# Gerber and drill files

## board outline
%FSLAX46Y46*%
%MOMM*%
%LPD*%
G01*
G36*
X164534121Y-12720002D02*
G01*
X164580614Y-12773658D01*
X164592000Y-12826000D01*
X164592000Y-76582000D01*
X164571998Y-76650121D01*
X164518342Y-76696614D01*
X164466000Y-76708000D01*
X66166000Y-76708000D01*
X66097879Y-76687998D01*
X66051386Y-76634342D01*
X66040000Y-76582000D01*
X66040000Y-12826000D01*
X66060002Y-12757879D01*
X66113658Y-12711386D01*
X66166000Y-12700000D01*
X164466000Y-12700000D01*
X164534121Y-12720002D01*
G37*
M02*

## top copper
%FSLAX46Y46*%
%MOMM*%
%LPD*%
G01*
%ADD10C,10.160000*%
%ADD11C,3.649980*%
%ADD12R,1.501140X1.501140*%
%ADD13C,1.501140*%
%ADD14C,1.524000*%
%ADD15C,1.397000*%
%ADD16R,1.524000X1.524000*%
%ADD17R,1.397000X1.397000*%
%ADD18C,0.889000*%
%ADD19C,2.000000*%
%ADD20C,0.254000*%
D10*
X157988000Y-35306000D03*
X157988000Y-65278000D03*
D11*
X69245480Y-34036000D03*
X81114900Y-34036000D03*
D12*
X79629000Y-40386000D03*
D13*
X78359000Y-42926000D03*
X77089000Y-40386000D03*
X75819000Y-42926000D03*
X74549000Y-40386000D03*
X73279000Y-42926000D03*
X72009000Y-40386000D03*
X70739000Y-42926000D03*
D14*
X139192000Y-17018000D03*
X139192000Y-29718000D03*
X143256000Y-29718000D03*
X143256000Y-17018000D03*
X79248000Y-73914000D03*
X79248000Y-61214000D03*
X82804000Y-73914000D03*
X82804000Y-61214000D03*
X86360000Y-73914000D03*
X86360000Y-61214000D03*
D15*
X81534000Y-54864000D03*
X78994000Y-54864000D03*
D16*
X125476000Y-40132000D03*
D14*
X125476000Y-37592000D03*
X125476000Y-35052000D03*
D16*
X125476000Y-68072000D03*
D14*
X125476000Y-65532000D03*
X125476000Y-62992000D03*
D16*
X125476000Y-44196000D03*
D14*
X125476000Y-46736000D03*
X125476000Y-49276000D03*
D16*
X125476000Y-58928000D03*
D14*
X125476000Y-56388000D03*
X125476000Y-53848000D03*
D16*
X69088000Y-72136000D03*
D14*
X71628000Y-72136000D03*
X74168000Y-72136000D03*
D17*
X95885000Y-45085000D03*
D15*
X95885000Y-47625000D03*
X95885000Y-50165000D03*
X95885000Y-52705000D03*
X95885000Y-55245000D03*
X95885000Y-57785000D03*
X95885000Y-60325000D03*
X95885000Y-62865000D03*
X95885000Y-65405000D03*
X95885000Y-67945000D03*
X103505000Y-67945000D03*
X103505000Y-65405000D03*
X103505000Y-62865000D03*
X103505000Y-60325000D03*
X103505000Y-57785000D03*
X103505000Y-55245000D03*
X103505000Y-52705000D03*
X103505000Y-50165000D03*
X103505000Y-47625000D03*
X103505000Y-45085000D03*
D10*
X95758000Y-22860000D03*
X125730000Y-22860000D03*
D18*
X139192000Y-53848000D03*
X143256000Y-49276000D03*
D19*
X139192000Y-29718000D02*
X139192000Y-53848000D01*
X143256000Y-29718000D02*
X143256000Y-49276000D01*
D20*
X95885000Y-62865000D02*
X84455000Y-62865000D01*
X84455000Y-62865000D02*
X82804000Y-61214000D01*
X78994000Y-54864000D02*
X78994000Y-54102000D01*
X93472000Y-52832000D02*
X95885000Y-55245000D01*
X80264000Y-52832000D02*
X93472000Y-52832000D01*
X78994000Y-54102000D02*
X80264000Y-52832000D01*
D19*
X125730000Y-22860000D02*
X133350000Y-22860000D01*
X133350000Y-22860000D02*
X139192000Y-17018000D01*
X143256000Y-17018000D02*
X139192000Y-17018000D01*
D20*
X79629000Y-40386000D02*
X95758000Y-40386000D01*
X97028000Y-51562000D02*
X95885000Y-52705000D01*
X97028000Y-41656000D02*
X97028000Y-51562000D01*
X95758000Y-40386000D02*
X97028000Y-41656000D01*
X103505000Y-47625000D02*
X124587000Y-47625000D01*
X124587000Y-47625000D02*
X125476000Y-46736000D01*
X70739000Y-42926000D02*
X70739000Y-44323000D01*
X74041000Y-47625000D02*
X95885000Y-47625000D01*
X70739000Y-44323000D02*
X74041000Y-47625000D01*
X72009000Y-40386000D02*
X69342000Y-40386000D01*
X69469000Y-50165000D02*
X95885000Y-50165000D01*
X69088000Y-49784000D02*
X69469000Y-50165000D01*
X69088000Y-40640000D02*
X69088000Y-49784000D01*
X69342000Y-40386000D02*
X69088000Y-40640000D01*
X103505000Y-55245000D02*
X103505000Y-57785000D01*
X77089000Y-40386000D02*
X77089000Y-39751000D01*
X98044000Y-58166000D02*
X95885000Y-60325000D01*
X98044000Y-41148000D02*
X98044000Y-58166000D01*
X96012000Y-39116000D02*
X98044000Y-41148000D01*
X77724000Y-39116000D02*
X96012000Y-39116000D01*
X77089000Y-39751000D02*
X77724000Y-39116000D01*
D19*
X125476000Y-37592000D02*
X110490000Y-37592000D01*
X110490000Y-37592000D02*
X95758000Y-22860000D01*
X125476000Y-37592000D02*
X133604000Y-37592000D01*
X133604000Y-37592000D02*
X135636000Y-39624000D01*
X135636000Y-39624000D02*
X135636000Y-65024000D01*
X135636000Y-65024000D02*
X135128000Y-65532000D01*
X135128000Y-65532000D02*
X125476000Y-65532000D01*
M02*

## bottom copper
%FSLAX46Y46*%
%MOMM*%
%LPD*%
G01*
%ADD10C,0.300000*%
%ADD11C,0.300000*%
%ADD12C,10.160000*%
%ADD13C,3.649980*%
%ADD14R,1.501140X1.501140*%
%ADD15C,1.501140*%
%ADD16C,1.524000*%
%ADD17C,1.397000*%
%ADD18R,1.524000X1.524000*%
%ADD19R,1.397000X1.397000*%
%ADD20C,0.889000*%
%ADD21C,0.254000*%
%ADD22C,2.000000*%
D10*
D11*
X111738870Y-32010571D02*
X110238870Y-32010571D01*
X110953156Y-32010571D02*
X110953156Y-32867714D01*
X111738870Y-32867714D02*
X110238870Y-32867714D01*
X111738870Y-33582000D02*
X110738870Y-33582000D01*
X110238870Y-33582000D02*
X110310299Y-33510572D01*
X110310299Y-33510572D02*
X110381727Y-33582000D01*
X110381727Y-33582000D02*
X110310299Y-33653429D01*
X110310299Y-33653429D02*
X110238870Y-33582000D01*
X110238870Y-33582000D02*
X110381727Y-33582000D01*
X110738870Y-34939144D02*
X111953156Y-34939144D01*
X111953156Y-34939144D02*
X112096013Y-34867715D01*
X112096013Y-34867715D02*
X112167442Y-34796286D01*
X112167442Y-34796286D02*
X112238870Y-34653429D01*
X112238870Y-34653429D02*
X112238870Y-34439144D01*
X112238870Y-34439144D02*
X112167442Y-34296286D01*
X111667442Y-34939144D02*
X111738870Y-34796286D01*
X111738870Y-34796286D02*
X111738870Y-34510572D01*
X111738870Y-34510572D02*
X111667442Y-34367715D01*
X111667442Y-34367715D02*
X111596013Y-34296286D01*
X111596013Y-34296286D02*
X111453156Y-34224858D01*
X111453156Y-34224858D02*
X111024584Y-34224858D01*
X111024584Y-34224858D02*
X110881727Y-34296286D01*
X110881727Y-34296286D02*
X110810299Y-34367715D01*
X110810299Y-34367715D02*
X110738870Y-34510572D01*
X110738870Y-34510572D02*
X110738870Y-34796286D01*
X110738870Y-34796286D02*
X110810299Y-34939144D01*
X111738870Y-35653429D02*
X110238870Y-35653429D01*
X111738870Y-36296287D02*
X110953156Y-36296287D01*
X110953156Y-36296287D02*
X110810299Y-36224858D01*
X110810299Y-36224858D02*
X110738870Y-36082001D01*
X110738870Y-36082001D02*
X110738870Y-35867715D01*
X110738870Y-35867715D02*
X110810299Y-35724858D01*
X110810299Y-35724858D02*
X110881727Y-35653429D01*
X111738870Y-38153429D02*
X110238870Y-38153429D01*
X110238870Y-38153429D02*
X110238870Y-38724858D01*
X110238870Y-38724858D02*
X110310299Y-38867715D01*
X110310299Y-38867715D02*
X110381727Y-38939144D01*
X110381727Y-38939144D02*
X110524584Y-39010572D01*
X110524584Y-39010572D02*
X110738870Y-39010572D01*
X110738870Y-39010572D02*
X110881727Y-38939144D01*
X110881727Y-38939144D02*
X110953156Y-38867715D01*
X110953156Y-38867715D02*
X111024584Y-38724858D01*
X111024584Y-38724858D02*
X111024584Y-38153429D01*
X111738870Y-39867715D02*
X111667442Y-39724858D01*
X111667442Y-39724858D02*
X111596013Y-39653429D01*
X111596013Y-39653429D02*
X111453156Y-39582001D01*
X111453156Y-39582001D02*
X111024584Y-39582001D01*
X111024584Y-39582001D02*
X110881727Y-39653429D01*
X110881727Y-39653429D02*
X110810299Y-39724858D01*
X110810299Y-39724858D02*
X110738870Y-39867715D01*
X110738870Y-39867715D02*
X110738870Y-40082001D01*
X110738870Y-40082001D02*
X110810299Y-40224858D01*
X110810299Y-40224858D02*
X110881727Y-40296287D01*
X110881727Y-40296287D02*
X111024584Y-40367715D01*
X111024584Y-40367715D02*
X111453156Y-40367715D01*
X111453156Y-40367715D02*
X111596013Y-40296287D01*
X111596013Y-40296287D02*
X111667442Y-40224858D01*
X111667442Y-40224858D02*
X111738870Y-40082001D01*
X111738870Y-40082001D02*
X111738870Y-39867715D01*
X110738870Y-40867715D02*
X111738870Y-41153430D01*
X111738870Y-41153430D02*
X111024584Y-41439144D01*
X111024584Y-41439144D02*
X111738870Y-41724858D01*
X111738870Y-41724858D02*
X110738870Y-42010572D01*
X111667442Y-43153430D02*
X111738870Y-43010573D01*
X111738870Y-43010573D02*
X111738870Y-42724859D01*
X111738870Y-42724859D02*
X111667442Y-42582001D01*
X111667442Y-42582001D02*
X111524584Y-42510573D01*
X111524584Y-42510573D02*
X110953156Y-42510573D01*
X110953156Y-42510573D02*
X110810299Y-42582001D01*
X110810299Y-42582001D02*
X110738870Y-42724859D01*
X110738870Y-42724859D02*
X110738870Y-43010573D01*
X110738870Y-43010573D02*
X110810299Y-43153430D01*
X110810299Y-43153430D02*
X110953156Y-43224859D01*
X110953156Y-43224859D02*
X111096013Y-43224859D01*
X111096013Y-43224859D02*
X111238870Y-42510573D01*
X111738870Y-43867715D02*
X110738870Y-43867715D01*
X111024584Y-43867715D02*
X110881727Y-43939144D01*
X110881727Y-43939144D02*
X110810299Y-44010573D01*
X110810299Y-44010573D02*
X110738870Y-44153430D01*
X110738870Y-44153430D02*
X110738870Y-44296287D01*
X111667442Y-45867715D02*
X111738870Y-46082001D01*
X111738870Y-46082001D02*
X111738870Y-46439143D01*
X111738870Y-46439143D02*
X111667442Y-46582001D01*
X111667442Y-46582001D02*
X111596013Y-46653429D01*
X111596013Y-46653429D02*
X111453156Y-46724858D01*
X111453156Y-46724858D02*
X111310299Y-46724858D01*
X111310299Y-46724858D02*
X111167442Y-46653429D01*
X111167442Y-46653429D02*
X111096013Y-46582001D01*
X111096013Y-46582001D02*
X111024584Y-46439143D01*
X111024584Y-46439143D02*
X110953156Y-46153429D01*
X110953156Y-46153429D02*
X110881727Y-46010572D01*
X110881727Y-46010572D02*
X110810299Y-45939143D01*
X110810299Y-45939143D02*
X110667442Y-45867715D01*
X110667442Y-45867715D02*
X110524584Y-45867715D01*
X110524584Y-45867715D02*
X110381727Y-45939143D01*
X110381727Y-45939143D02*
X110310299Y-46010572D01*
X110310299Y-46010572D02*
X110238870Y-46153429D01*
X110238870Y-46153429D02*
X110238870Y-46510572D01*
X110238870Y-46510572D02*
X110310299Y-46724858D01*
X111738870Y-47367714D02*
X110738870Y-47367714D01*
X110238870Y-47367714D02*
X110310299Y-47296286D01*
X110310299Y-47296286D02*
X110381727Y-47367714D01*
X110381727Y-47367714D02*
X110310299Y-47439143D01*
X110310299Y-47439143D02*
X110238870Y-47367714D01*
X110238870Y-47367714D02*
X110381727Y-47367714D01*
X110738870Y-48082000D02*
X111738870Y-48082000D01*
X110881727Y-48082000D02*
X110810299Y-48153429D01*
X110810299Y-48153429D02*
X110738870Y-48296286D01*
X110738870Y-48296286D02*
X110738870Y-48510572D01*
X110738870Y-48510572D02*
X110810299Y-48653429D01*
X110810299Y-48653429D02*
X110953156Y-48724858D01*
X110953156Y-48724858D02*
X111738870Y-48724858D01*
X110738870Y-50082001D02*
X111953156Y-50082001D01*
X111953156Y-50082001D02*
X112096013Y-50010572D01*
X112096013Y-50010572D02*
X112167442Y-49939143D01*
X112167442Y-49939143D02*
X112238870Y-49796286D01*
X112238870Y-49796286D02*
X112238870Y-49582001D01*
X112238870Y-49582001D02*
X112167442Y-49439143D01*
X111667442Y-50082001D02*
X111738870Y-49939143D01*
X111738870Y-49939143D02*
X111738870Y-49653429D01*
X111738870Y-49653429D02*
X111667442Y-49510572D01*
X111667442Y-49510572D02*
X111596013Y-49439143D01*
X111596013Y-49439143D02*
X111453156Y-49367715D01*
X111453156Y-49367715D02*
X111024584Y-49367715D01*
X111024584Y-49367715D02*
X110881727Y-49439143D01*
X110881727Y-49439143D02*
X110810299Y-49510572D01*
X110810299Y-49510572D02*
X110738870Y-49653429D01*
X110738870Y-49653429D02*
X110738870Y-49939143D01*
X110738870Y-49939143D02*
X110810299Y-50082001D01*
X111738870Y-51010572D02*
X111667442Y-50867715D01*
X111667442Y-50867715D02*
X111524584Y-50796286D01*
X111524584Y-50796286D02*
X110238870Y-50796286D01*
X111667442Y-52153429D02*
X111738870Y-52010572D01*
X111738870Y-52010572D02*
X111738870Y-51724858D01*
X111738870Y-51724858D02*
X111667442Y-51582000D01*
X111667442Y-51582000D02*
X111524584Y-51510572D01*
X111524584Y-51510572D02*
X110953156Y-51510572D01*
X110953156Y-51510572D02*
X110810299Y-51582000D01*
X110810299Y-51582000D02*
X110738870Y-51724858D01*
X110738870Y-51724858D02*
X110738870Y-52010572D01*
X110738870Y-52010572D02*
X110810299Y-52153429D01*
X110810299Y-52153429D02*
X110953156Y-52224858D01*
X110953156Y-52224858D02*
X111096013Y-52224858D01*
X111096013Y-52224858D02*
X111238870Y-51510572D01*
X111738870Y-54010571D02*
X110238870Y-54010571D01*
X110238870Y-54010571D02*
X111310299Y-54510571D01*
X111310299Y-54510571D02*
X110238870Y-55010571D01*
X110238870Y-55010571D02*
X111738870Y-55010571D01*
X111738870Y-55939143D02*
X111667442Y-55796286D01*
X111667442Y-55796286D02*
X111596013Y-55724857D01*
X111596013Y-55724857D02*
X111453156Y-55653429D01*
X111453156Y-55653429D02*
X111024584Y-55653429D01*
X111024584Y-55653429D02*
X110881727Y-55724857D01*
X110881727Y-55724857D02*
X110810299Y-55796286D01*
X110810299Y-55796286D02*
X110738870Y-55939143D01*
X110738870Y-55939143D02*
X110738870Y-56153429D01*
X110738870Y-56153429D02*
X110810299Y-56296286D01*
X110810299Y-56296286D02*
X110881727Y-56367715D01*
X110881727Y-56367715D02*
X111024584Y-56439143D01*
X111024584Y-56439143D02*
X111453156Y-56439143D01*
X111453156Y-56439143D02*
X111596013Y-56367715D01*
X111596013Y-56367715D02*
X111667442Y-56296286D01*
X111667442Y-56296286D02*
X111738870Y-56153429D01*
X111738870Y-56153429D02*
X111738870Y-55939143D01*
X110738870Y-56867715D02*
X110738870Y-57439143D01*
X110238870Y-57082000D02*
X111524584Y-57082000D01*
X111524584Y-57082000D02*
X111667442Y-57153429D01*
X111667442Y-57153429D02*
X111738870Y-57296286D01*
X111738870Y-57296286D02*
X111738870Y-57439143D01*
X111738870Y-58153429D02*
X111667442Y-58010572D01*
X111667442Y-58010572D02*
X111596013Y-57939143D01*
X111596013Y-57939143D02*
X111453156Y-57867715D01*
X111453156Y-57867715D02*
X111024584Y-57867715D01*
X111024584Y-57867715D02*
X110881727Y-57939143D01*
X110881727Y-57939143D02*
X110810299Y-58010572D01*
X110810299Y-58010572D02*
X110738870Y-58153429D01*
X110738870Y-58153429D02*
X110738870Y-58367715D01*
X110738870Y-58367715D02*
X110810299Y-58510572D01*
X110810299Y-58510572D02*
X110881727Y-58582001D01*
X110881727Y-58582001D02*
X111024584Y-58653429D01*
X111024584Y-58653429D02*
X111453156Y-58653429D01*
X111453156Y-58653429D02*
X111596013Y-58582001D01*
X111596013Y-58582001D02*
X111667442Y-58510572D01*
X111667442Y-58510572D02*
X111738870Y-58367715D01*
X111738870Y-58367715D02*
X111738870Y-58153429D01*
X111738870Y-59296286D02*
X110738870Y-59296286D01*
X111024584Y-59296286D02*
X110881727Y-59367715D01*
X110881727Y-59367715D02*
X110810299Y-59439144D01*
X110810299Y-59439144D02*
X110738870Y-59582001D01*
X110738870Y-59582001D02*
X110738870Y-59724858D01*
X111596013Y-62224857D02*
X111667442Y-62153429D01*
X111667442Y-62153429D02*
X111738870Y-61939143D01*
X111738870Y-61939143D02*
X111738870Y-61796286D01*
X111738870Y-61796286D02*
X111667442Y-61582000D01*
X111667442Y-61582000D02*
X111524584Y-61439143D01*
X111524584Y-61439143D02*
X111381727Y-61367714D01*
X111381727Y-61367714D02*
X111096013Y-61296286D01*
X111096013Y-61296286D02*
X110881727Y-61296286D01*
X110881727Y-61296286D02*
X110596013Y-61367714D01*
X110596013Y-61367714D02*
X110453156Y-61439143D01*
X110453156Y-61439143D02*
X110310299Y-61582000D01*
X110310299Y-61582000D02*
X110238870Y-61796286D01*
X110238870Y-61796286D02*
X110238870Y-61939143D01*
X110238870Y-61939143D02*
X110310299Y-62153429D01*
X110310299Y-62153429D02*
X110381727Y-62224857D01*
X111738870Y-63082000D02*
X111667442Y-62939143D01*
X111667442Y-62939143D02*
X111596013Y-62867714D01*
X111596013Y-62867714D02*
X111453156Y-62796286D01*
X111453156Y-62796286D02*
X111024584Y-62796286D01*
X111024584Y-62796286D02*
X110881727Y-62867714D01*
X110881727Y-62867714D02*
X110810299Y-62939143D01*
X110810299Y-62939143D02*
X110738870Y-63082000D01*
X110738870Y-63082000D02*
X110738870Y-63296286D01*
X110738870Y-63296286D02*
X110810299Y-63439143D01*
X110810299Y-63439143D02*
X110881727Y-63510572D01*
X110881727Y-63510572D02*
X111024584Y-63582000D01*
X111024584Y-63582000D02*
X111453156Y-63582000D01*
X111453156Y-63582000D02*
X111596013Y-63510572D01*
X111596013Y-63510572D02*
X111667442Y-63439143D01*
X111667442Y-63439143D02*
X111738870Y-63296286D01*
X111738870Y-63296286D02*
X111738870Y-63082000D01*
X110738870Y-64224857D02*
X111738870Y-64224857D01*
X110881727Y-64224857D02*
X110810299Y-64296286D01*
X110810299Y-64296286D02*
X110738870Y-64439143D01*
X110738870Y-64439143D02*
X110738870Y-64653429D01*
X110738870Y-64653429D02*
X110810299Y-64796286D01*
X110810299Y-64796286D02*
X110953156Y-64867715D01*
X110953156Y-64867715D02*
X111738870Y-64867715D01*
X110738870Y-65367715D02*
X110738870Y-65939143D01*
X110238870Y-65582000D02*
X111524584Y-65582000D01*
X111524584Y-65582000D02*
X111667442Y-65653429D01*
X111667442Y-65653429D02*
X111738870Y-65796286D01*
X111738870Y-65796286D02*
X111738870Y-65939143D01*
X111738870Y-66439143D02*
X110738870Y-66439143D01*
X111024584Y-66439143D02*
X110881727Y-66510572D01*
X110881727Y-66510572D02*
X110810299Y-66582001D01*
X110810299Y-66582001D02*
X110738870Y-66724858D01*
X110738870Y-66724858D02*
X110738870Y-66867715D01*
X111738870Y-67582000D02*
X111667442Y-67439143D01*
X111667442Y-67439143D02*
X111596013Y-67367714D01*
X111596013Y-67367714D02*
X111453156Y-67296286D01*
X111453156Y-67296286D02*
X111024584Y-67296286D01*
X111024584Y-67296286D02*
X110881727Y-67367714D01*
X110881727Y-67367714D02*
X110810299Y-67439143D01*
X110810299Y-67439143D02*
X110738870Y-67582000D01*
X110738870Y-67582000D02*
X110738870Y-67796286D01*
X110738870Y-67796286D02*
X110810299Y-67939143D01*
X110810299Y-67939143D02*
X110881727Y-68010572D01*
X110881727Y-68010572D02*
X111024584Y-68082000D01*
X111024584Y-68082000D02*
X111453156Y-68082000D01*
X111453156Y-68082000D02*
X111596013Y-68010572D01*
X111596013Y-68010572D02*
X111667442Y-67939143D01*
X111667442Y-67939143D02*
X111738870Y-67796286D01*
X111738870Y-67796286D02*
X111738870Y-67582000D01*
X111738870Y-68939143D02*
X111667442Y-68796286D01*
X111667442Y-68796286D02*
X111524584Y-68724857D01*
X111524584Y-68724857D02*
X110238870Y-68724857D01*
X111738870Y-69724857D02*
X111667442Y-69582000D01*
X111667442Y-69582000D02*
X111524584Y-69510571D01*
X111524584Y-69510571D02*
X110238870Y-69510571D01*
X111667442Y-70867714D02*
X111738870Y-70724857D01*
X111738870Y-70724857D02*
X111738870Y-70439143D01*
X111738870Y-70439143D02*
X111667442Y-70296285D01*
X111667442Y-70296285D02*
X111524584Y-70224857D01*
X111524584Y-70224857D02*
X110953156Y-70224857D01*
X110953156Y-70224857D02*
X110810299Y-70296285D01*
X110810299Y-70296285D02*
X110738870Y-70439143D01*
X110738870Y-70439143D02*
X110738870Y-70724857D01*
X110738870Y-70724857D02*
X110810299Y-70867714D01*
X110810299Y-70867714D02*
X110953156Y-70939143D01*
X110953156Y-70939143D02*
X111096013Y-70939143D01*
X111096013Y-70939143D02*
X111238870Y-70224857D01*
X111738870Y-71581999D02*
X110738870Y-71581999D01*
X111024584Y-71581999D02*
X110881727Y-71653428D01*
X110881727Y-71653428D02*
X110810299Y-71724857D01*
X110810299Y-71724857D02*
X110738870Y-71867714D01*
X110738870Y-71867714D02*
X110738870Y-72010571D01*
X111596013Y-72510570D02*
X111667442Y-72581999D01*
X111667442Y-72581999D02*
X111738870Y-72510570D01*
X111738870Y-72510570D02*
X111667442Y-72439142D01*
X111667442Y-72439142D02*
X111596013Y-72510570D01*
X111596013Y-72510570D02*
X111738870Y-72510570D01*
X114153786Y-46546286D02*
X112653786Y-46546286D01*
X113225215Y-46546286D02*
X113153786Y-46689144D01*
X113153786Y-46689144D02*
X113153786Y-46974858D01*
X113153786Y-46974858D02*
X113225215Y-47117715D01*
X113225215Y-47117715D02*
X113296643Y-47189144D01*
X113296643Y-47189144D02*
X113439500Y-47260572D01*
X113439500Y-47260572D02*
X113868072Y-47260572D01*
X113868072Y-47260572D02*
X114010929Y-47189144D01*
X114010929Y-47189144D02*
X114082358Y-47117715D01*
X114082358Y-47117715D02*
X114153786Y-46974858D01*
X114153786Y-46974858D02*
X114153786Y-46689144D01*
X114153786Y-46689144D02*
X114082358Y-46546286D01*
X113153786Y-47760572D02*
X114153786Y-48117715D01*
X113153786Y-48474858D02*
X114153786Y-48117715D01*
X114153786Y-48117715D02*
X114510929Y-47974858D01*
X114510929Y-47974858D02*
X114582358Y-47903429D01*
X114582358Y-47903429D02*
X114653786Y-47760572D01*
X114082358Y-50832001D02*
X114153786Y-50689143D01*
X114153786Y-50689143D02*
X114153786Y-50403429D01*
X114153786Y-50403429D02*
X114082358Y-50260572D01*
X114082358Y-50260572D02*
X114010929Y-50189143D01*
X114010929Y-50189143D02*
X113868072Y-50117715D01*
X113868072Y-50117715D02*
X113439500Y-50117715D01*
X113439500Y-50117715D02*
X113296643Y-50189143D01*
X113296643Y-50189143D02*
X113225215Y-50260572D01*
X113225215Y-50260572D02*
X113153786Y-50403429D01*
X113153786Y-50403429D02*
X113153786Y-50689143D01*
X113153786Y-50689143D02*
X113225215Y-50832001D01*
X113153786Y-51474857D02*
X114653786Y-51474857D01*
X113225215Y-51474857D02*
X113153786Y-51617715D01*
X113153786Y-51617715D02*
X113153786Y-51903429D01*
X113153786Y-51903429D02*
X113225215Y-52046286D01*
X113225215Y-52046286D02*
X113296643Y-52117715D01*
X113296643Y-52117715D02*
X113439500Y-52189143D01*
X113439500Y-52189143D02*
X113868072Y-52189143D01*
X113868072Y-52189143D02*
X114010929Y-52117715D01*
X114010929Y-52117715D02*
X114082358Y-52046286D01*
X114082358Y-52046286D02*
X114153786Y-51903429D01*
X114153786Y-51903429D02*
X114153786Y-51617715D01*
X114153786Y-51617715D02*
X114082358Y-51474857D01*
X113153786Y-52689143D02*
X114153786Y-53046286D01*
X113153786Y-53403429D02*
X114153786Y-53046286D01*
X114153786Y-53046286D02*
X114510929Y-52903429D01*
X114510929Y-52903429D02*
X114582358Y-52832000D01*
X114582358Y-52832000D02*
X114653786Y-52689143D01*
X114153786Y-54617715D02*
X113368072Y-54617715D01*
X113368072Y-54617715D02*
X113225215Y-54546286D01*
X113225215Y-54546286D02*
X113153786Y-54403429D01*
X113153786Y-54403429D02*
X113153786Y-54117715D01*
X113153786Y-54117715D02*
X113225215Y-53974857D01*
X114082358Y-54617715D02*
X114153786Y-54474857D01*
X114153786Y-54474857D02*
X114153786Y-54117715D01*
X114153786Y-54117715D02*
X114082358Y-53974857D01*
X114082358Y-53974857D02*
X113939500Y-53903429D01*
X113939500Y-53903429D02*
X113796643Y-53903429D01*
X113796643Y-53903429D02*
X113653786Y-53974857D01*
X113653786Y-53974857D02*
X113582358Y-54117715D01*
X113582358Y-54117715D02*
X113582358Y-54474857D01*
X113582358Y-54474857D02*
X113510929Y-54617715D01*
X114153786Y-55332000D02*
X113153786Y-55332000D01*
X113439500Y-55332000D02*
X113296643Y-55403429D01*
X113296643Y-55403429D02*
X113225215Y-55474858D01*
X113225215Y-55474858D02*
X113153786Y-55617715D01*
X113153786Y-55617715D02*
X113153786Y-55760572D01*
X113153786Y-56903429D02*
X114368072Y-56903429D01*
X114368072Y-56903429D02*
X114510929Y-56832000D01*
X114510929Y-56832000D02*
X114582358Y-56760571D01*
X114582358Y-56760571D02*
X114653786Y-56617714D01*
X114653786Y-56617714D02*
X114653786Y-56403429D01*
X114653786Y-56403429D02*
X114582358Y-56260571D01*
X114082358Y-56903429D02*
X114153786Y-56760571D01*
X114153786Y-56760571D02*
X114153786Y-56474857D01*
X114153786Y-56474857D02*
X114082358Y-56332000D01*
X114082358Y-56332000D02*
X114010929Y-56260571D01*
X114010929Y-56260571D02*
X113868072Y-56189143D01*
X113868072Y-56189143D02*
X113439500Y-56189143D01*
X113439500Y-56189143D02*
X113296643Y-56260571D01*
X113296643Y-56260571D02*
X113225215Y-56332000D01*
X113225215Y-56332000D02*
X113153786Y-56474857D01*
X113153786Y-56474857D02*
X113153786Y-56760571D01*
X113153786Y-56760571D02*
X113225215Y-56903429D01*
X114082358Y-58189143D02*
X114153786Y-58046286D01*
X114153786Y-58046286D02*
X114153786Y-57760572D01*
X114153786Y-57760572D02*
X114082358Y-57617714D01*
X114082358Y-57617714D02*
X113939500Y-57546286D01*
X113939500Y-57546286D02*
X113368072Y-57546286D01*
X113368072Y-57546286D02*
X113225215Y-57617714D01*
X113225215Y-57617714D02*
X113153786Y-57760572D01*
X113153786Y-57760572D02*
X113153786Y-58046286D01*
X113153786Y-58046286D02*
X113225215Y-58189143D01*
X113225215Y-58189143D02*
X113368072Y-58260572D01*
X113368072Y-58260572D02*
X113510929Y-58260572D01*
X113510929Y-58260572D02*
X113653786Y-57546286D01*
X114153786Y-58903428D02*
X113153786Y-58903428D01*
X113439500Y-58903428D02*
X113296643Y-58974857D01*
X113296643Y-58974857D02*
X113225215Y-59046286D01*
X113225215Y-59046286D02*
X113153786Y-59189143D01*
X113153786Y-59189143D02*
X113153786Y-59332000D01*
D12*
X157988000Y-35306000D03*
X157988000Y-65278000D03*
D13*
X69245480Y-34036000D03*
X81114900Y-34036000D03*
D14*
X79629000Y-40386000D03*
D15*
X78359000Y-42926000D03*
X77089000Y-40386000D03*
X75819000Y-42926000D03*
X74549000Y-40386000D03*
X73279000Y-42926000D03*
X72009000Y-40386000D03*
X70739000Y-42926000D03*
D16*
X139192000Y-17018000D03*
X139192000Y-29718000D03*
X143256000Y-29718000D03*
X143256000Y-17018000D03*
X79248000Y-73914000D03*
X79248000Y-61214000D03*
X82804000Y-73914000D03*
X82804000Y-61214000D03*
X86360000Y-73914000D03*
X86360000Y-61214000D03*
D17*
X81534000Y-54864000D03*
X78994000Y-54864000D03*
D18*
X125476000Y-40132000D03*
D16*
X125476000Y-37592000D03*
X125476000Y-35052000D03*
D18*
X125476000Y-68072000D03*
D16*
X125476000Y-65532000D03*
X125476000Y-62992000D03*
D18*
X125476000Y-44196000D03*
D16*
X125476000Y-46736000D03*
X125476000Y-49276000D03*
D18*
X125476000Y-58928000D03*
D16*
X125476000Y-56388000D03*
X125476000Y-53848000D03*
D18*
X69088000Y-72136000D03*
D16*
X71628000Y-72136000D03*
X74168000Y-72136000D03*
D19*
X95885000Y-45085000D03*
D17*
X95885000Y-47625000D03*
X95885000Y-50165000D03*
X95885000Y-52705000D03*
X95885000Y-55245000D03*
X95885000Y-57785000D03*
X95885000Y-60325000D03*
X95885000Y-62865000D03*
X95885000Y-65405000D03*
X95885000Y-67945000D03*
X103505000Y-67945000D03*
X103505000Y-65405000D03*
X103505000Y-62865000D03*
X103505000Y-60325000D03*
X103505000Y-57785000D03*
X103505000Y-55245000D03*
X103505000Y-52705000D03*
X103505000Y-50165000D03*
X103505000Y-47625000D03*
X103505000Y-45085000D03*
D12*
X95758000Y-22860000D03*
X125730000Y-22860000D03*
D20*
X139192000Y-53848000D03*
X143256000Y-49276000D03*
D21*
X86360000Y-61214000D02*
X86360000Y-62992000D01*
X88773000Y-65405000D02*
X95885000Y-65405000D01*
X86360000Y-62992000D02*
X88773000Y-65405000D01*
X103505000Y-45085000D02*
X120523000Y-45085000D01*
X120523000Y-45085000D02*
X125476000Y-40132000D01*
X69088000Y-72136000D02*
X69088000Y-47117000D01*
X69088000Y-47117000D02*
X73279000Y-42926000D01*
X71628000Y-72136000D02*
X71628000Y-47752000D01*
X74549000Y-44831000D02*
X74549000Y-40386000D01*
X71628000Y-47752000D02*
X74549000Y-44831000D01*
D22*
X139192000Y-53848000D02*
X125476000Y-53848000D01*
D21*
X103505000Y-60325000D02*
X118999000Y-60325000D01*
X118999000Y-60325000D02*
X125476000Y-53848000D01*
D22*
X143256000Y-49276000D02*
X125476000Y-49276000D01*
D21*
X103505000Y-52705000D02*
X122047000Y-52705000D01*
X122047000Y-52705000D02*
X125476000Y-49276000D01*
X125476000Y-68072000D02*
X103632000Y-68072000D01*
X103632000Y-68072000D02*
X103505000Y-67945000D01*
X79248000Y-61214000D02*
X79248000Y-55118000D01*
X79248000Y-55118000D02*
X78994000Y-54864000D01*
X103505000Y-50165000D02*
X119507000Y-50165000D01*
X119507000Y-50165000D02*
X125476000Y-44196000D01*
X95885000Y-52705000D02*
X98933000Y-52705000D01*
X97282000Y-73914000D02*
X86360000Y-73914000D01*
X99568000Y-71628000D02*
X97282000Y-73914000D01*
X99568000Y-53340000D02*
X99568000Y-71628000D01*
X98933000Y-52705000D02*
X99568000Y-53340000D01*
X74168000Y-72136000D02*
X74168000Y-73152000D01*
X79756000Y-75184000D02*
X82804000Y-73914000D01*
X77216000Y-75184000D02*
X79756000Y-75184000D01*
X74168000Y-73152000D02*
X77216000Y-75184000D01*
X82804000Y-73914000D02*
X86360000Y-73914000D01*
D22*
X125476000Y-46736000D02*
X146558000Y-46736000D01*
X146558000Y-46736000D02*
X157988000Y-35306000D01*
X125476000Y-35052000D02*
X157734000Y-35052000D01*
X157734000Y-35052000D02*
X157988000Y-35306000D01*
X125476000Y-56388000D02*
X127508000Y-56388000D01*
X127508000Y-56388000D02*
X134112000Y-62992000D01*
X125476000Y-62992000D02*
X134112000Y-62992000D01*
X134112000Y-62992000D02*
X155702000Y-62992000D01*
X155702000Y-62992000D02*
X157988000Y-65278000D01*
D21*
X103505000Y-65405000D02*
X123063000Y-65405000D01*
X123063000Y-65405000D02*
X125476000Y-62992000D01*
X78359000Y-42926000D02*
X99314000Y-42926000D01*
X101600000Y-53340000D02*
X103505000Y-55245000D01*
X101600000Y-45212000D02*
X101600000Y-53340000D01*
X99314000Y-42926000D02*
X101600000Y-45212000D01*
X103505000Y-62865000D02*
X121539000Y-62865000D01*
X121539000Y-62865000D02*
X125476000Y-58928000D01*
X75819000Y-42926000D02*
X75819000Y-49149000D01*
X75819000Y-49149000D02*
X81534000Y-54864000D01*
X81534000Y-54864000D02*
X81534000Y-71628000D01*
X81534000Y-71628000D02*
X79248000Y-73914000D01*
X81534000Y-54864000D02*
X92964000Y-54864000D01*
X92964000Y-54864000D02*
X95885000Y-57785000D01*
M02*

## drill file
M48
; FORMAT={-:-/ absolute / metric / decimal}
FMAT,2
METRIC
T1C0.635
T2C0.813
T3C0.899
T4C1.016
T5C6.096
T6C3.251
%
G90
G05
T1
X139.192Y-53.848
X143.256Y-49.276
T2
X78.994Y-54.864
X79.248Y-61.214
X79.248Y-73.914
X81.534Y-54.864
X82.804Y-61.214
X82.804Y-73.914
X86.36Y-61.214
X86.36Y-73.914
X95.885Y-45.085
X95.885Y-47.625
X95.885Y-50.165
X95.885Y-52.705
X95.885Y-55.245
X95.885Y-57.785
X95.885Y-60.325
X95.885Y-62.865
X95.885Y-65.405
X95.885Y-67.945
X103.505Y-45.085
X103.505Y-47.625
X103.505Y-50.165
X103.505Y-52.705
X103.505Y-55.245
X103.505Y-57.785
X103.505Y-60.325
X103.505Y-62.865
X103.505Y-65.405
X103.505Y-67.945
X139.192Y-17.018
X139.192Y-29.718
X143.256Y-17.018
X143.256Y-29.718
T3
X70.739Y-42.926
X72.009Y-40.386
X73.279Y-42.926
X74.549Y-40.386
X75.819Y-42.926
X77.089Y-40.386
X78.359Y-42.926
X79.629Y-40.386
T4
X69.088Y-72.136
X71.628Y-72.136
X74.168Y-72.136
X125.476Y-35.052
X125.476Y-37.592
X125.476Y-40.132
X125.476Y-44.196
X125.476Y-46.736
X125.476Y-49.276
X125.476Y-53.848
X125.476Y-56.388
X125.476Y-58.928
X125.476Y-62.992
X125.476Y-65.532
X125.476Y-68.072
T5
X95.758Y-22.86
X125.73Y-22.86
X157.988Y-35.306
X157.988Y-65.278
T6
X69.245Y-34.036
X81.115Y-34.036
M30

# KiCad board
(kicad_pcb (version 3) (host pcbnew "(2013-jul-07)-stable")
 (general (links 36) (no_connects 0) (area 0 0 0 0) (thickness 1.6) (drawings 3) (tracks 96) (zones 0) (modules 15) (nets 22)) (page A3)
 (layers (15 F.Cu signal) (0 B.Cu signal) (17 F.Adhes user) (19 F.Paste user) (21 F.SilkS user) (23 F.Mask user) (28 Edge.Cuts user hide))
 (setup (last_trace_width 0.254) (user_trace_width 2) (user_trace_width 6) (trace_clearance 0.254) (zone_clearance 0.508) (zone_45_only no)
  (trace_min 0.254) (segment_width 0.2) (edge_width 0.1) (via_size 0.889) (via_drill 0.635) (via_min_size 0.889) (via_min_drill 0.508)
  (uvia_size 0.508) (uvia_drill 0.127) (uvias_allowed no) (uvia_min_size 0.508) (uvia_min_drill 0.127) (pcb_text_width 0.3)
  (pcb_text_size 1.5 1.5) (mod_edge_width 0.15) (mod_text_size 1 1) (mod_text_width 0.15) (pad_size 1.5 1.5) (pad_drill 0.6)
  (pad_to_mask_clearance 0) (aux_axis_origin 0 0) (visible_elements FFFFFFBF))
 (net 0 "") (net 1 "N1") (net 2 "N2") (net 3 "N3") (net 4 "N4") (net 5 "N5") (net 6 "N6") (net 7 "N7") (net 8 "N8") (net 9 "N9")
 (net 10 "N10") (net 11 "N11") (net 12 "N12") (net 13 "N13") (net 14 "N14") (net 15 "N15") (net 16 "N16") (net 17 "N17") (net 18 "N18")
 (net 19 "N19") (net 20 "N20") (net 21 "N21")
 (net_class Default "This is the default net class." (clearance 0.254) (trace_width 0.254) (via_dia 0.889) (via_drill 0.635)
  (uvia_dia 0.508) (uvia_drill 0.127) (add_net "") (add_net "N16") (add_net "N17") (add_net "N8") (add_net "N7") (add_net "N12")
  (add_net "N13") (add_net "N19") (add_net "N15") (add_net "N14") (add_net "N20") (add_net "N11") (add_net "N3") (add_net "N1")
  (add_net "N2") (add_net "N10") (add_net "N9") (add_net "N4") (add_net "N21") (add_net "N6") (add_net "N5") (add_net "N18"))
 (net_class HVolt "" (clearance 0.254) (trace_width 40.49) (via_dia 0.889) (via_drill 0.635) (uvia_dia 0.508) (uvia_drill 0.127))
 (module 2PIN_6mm (layer F.Cu) (at 157.988 50.292 270)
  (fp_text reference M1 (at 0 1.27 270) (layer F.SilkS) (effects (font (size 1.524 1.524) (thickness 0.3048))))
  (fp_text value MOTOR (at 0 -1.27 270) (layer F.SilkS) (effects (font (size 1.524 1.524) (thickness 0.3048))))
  (pad 1 thru_hole circle (at -14.986 0 270) (size 10.16 10.16) (drill 6.096) (layers *.Cu *.Mask F.SilkS) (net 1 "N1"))
  (pad 2 thru_hole circle (at 14.986 0 270) (size 10.16 10.16) (drill 6.096) (layers *.Cu *.Mask F.SilkS) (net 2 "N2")))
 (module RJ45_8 (layer F.Cu) (at 75.184 34.036 180)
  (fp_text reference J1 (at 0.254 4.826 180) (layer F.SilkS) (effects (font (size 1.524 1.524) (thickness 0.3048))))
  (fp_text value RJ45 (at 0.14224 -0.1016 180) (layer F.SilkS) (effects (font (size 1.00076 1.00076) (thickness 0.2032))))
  (pad Hole np_thru_hole circle (at 5.93852 0 180) (size 3.64998 3.64998) (drill 3.2512) (layers *.Cu *.SilkS *.Mask))
  (pad Hole np_thru_hole circle (at -5.9309 0 180) (size 3.64998 3.64998) (drill 3.2512) (layers *.Cu *.SilkS *.Mask))
  (pad 1 thru_hole rect (at -4.445 -6.35 180) (size 1.50114 1.50114) (drill 0.89916) (layers *.Cu *.Mask F.SilkS) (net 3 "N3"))
  (pad 2 thru_hole circle (at -3.175 -8.89 180) (size 1.50114 1.50114) (drill 0.89916) (layers *.Cu *.Mask F.SilkS) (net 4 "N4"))
  (pad 3 thru_hole circle (at -1.905 -6.35 180) (size 1.50114 1.50114) (drill 0.89916) (layers *.Cu *.Mask F.SilkS) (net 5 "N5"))
  (pad 4 thru_hole circle (at -0.635 -8.89 180) (size 1.50114 1.50114) (drill 0.89916) (layers *.Cu *.Mask F.SilkS) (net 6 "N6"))
  (pad 5 thru_hole circle (at 0.635 -6.35 180) (size 1.50114 1.50114) (drill 0.89916) (layers *.Cu *.Mask F.SilkS) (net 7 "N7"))
  (pad 6 thru_hole circle (at 1.905 -8.89 180) (size 1.50114 1.50114) (drill 0.89916) (layers *.Cu *.Mask F.SilkS) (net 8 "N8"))
  (pad 7 thru_hole circle (at 3.175 -6.35 180) (size 1.50114 1.50114) (drill 0.89916) (layers *.Cu *.Mask F.SilkS) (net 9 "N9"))
  (pad 8 thru_hole circle (at 4.445 -8.89 180) (size 1.50114 1.50114) (drill 0.89916) (layers *.Cu *.Mask F.SilkS) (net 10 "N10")))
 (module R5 (layer F.Cu) (at 139.192 23.368 270) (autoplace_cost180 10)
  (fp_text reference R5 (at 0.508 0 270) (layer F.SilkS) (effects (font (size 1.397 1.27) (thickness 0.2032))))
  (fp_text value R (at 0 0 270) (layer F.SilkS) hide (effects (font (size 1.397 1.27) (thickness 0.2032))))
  (pad 1 thru_hole circle (at -6.35 0 270) (size 1.524 1.524) (drill 0.8128) (layers *.Cu *.Mask F.SilkS) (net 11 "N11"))
  (pad 2 thru_hole circle (at 6.35 0 270) (size 1.524 1.524) (drill 0.8128) (layers *.Cu *.Mask F.SilkS) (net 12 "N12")))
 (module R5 (layer F.Cu) (at 143.256 23.368 90) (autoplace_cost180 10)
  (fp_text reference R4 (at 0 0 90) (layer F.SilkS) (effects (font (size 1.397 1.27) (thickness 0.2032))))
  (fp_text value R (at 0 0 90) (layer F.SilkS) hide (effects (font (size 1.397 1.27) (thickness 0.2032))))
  (pad 1 thru_hole circle (at -6.35 0 90) (size 1.524 1.524) (drill 0.8128) (layers *.Cu *.Mask F.SilkS) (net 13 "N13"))
  (pad 2 thru_hole circle (at 6.35 0 90) (size 1.524 1.524) (drill 0.8128) (layers *.Cu *.Mask F.SilkS) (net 11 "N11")))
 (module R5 (layer F.Cu) (at 79.248 67.564 90) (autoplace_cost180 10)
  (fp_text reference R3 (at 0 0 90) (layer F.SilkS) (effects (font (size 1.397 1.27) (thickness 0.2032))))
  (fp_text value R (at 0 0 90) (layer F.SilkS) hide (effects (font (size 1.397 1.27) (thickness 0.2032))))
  (pad 1 thru_hole circle (at -6.35 0 90) (size 1.524 1.524) (drill 0.8128) (layers *.Cu *.Mask F.SilkS) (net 6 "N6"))
  (pad 2 thru_hole circle (at 6.35 0 90) (size 1.524 1.524) (drill 0.8128) (layers *.Cu *.Mask F.SilkS) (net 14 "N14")))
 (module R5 (layer F.Cu) (at 82.804 67.564 90) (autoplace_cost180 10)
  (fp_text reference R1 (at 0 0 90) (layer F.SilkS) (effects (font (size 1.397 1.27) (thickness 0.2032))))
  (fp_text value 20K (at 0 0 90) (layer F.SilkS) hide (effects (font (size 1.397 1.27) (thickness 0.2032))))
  (pad 1 thru_hole circle (at -6.35 0 90) (size 1.524 1.524) (drill 0.8128) (layers *.Cu *.Mask F.SilkS) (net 3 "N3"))
  (pad 2 thru_hole circle (at 6.35 0 90) (size 1.524 1.524) (drill 0.8128) (layers *.Cu *.Mask F.SilkS) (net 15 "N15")))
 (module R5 (layer F.Cu) (at 86.36 67.564 90) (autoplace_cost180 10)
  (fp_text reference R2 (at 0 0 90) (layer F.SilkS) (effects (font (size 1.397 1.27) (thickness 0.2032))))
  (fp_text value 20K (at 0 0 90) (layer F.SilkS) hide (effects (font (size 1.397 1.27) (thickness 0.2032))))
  (pad 1 thru_hole circle (at -6.35 0 90) (size 1.524 1.524) (drill 0.8128) (layers *.Cu *.Mask F.SilkS) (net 3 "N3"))
  (pad 2 thru_hole circle (at 6.35 0 90) (size 1.524 1.524) (drill 0.8128) (layers *.Cu *.Mask F.SilkS) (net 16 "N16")))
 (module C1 (layer F.Cu) (at 80.264 54.864 180)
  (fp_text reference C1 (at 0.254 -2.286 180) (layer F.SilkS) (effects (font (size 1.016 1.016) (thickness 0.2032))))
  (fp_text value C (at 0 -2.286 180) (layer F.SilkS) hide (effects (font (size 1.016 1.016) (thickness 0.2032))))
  (pad 1 thru_hole circle (at -1.27 0 180) (size 1.397 1.397) (drill 0.8128) (layers *.Cu *.Mask F.SilkS) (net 6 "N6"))
  (pad 2 thru_hole circle (at 1.27 0 180) (size 1.397 1.397) (drill 0.8128) (layers *.Cu *.Mask F.SilkS) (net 14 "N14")))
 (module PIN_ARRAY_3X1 (layer F.Cu) (at 125.476 37.592 90)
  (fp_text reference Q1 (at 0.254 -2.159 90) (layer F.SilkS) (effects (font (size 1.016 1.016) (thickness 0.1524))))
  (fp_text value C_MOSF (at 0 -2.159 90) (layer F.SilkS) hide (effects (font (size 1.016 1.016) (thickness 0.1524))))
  (pad 1 thru_hole rect (at -2.54 0 90) (size 1.524 1.524) (drill 1.016) (layers *.Cu *.Mask F.SilkS) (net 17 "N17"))
  (pad 2 thru_hole circle (at 0 0 90) (size 1.524 1.524) (drill 1.016) (layers *.Cu *.Mask F.SilkS) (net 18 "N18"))
  (pad 3 thru_hole circle (at 2.54 0 90) (size 1.524 1.524) (drill 1.016) (layers *.Cu *.Mask F.SilkS) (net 1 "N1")))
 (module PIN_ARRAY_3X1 (layer F.Cu) (at 125.476 65.532 90)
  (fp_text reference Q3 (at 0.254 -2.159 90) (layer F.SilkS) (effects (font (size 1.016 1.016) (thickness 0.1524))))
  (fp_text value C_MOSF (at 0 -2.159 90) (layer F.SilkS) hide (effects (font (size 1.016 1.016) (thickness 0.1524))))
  (pad 1 thru_hole rect (at -2.54 0 90) (size 1.524 1.524) (drill 1.016) (layers *.Cu *.Mask F.SilkS) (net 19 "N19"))
  (pad 2 thru_hole circle (at 0 0 90) (size 1.524 1.524) (drill 1.016) (layers *.Cu *.Mask F.SilkS) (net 18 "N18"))
  (pad 3 thru_hole circle (at 2.54 0 90) (size 1.524 1.524) (drill 1.016) (layers *.Cu *.Mask F.SilkS) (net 2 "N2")))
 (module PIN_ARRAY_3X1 (layer F.Cu) (at 125.476 46.736 270)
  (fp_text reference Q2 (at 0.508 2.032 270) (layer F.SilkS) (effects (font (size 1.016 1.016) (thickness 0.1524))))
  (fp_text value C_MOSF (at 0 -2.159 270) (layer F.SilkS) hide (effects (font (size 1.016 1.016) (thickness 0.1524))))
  (pad 1 thru_hole rect (at -2.54 0 270) (size 1.524 1.524) (drill 1.016) (layers *.Cu *.Mask F.SilkS) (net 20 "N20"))
  (pad 2 thru_hole circle (at 0 0 270) (size 1.524 1.524) (drill 1.016) (layers *.Cu *.Mask F.SilkS) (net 1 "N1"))
  (pad 3 thru_hole circle (at 2.54 0 270) (size 1.524 1.524) (drill 1.016) (layers *.Cu *.Mask F.SilkS) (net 13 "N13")))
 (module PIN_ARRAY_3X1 (layer F.Cu) (at 125.476 56.388 90)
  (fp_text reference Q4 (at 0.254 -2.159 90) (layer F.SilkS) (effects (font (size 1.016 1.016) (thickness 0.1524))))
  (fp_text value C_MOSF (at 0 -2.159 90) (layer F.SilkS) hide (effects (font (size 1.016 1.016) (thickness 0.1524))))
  (pad 1 thru_hole rect (at -2.54 0 90) (size 1.524 1.524) (drill 1.016) (layers *.Cu *.Mask F.SilkS) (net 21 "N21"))
  (pad 2 thru_hole circle (at 0 0 90) (size 1.524 1.524) (drill 1.016) (layers *.Cu *.Mask F.SilkS) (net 2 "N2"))
  (pad 3 thru_hole circle (at 2.54 0 90) (size 1.524 1.524) (drill 1.016) (layers *.Cu *.Mask F.SilkS) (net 12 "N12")))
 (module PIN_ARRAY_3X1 (layer F.Cu) (at 71.628 72.136)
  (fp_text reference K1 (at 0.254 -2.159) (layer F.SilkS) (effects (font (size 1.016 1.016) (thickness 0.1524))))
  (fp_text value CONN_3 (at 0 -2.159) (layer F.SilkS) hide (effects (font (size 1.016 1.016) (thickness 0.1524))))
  (pad 1 thru_hole rect (at -2.54 0) (size 1.524 1.524) (drill 1.016) (layers *.Cu *.Mask F.SilkS) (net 8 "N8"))
  (pad 2 thru_hole circle (at 0 0) (size 1.524 1.524) (drill 1.016) (layers *.Cu *.Mask F.SilkS) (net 7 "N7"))
  (pad 3 thru_hole circle (at 2.54 0) (size 1.524 1.524) (drill 1.016) (layers *.Cu *.Mask F.SilkS) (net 3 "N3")))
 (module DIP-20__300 (layer F.Cu) (at 99.695 56.515 270)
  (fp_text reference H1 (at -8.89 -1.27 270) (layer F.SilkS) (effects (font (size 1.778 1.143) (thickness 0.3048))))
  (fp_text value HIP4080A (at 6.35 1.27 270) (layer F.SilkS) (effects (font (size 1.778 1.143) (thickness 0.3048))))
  (pad 1 thru_hole rect (at -11.43 3.81 270) (size 1.397 1.397) (drill 0.8128) (layers *.Cu *.Mask F.SilkS))
  (pad 2 thru_hole circle (at -8.89 3.81 270) (size 1.397 1.397) (drill 0.8128) (layers *.Cu *.Mask F.SilkS) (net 10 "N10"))
  (pad 3 thru_hole circle (at -6.35 3.81 270) (size 1.397 1.397) (drill 0.8128) (layers *.Cu *.Mask F.SilkS) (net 9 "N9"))
  (pad 4 thru_hole circle (at -3.81 3.81 270) (size 1.397 1.397) (drill 0.8128) (layers *.Cu *.Mask F.SilkS) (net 3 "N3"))
  (pad 5 thru_hole circle (at -1.27 3.81 270) (size 1.397 1.397) (drill 0.8128) (layers *.Cu *.Mask F.SilkS) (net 14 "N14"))
  (pad 6 thru_hole circle (at 1.27 3.81 270) (size 1.397 1.397) (drill 0.8128) (layers *.Cu *.Mask F.SilkS) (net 6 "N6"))
  (pad 7 thru_hole circle (at 3.81 3.81 270) (size 1.397 1.397) (drill 0.8128) (layers *.Cu *.Mask F.SilkS) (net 5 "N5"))
  (pad 8 thru_hole circle (at 6.35 3.81 270) (size 1.397 1.397) (drill 0.8128) (layers *.Cu *.Mask F.SilkS) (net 15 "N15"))
  (pad 9 thru_hole circle (at 8.89 3.81 270) (size 1.397 1.397) (drill 0.8128) (layers *.Cu *.Mask F.SilkS) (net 16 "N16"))
  (pad 10 thru_hole circle (at 11.43 3.81 270) (size 1.397 1.397) (drill 0.8128) (layers *.Cu *.Mask F.SilkS))
  (pad 11 thru_hole circle (at 11.43 -3.81 270) (size 1.397 1.397) (drill 0.8128) (layers *.Cu *.Mask F.SilkS) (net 19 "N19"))
  (pad 12 thru_hole circle (at 8.89 -3.81 270) (size 1.397 1.397) (drill 0.8128) (layers *.Cu *.Mask F.SilkS) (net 2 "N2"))
  (pad 13 thru_hole circle (at 6.35 -3.81 270) (size 1.397 1.397) (drill 0.8128) (layers *.Cu *.Mask F.SilkS) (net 21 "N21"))
  (pad 14 thru_hole circle (at 3.81 -3.81 270) (size 1.397 1.397) (drill 0.8128) (layers *.Cu *.Mask F.SilkS) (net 12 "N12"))
  (pad 15 thru_hole circle (at 1.27 -3.81 270) (size 1.397 1.397) (drill 0.8128) (layers *.Cu *.Mask F.SilkS) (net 4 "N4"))
  (pad 16 thru_hole circle (at -1.27 -3.81 270) (size 1.397 1.397) (drill 0.8128) (layers *.Cu *.Mask F.SilkS) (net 4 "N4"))
  (pad 17 thru_hole circle (at -3.81 -3.81 270) (size 1.397 1.397) (drill 0.8128) (layers *.Cu *.Mask F.SilkS) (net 13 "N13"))
  (pad 18 thru_hole circle (at -6.35 -3.81 270) (size 1.397 1.397) (drill 0.8128) (layers *.Cu *.Mask F.SilkS) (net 20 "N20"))
  (pad 19 thru_hole circle (at -8.89 -3.81 270) (size 1.397 1.397) (drill 0.8128) (layers *.Cu *.Mask F.SilkS) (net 1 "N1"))
  (pad 20 thru_hole circle (at -11.43 -3.81 270) (size 1.397 1.397) (drill 0.8128) (layers *.Cu *.Mask F.SilkS) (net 17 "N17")))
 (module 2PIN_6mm (layer F.Cu) (at 110.744 22.86)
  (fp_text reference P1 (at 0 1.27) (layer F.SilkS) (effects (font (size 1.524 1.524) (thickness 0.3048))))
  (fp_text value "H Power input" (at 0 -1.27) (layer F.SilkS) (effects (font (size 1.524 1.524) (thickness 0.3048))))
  (pad 1 thru_hole circle (at -14.986 0) (size 10.16 10.16) (drill 6.096) (layers *.Cu *.Mask F.SilkS) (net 18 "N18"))
  (pad 2 thru_hole circle (at 14.986 0) (size 10.16 10.16) (drill 6.096) (layers *.Cu *.Mask F.SilkS) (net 11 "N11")))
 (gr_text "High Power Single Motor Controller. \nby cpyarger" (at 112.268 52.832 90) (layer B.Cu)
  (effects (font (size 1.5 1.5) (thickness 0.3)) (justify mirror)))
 (segment (start 86.36 61.214) (end 86.36 62.992) (width 0.254) (layer B.Cu) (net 16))
 (segment (start 88.773 65.405) (end 95.885 65.405) (width 0.254) (layer B.Cu) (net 16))
 (segment (start 86.36 62.992) (end 88.773 65.405) (width 0.254) (layer B.Cu) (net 16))
 (segment (start 103.505 45.085) (end 120.523 45.085) (width 0.254) (layer B.Cu) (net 17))
 (segment (start 120.523 45.085) (end 125.476 40.132) (width 0.254) (layer B.Cu) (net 17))
 (segment (start 69.088 72.136) (end 69.088 47.117) (width 0.254) (layer B.Cu) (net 8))
 (segment (start 69.088 47.117) (end 73.279 42.926) (width 0.254) (layer B.Cu) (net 8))
 (segment (start 71.628 72.136) (end 71.628 47.752) (width 0.254) (layer B.Cu) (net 7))
 (segment (start 74.549 44.831) (end 74.549 40.386) (width 0.254) (layer B.Cu) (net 7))
 (segment (start 71.628 47.752) (end 74.549 44.831) (width 0.254) (layer B.Cu) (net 7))
 (segment (start 139.192 29.718) (end 139.192 53.848) (width 2) (layer F.Cu) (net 12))
 (segment (start 139.192 53.848) (end 125.476 53.848) (width 2) (layer B.Cu) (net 12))
 (via (at 139.192 53.848) (size 0.889) (layers F.Cu B.Cu) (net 12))
 (segment (start 103.505 60.325) (end 118.999 60.325) (width 0.254) (layer B.Cu) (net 12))
 (segment (start 118.999 60.325) (end 125.476 53.848) (width 0.254) (layer B.Cu) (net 12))
 (segment (start 143.256 29.718) (end 143.256 49.276) (width 2) (layer F.Cu) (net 13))
 (segment (start 143.256 49.276) (end 125.476 49.276) (width 2) (layer B.Cu) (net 13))
 (via (at 143.256 49.276) (size 0.889) (layers F.Cu B.Cu) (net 13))
 (segment (start 103.505 52.705) (end 122.047 52.705) (width 0.254) (layer B.Cu) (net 13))
 (segment (start 122.047 52.705) (end 125.476 49.276) (width 0.254) (layer B.Cu) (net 13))
 (segment (start 125.476 68.072) (end 103.632 68.072) (width 0.254) (layer B.Cu) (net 19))
 (segment (start 103.632 68.072) (end 103.505 67.945) (width 0.254) (layer B.Cu) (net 19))
 (segment (start 95.885 62.865) (end 84.455 62.865) (width 0.254) (layer F.Cu) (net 15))
 (segment (start 84.455 62.865) (end 82.804 61.214) (width 0.254) (layer F.Cu) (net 15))
 (segment (start 78.994 54.864) (end 78.994 54.102) (width 0.254) (layer F.Cu) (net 14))
 (segment (start 93.472 52.832) (end 95.885 55.245) (width 0.254) (layer F.Cu) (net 14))
 (segment (start 80.264 52.832) (end 93.472 52.832) (width 0.254) (layer F.Cu) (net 14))
 (segment (start 78.994 54.102) (end 80.264 52.832) (width 0.254) (layer F.Cu) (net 14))
 (segment (start 79.248 61.214) (end 79.248 55.118) (width 0.254) (layer B.Cu) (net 14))
 (segment (start 79.248 55.118) (end 78.994 54.864) (width 0.254) (layer B.Cu) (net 14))
 (segment (start 103.505 50.165) (end 119.507 50.165) (width 0.254) (layer B.Cu) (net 20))
 (segment (start 119.507 50.165) (end 125.476 44.196) (width 0.254) (layer B.Cu) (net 20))
 (segment (start 125.73 22.86) (end 133.35 22.86) (width 2) (layer F.Cu) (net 11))
 (segment (start 133.35 22.86) (end 139.192 17.018) (width 2) (layer F.Cu) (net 11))
 (segment (start 143.256 17.018) (end 139.192 17.018) (width 2) (layer F.Cu) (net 11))
 (segment (start 95.885 52.705) (end 98.933 52.705) (width 0.254) (layer B.Cu) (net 3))
 (segment (start 97.282 73.914) (end 86.36 73.914) (width 0.254) (layer B.Cu) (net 3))
 (segment (start 99.568 71.628) (end 97.282 73.914) (width 0.254) (layer B.Cu) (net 3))
 (segment (start 99.568 53.34) (end 99.568 71.628) (width 0.254) (layer B.Cu) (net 3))
 (segment (start 98.933 52.705) (end 99.568 53.34) (width 0.254) (layer B.Cu) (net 3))
 (segment (start 79.629 40.386) (end 95.758 40.386) (width 0.254) (layer F.Cu) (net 3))
 (segment (start 97.028 51.562) (end 95.885 52.705) (width 0.254) (layer F.Cu) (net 3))
 (segment (start 97.028 41.656) (end 97.028 51.562) (width 0.254) (layer F.Cu) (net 3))
 (segment (start 95.758 40.386) (end 97.028 41.656) (width 0.254) (layer F.Cu) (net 3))
 (segment (start 74.168 72.136) (end 74.168 73.152) (width 0.254) (layer B.Cu) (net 3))
 (segment (start 79.756 75.184) (end 82.804 73.914) (width 0.254) (layer B.Cu) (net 3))
 (segment (start 77.216 75.184) (end 79.756 75.184) (width 0.254) (layer B.Cu) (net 3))
 (segment (start 74.168 73.152) (end 77.216 75.184) (width 0.254) (layer B.Cu) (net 3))
 (segment (start 82.804 73.914) (end 86.36 73.914) (width 0.254) (layer B.Cu) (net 3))
 (segment (start 125.476 46.736) (end 146.558 46.736) (width 2) (layer B.Cu) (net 1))
 (segment (start 146.558 46.736) (end 157.988 35.306) (width 2) (layer B.Cu) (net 1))
 (segment (start 125.476 35.052) (end 157.734 35.052) (width 2) (layer B.Cu) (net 1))
 (segment (start 157.734 35.052) (end 157.988 35.306) (width 2) (layer B.Cu) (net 1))
 (segment (start 103.505 47.625) (end 124.587 47.625) (width 0.254) (layer F.Cu) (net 1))
 (segment (start 124.587 47.625) (end 125.476 46.736) (width 0.254) (layer F.Cu) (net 1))
 (segment (start 125.476 56.388) (end 127.508 56.388) (width 2) (layer B.Cu) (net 2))
 (segment (start 127.508 56.388) (end 134.112 62.992) (width 2) (layer B.Cu) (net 2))
 (segment (start 125.476 62.992) (end 134.112 62.992) (width 2) (layer B.Cu) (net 2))
 (segment (start 134.112 62.992) (end 155.702 62.992) (width 2) (layer B.Cu) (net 2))
 (segment (start 155.702 62.992) (end 157.988 65.278) (width 2) (layer B.Cu) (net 2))
 (segment (start 103.505 65.405) (end 123.063 65.405) (width 0.254) (layer B.Cu) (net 2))
 (segment (start 123.063 65.405) (end 125.476 62.992) (width 0.254) (layer B.Cu) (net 2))
 (segment (start 70.739 42.926) (end 70.739 44.323) (width 0.254) (layer F.Cu) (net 10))
 (segment (start 74.041 47.625) (end 95.885 47.625) (width 0.254) (layer F.Cu) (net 10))
 (segment (start 70.739 44.323) (end 74.041 47.625) (width 0.254) (layer F.Cu) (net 10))
 (segment (start 72.009 40.386) (end 69.342 40.386) (width 0.254) (layer F.Cu) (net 9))
 (segment (start 69.469 50.165) (end 95.885 50.165) (width 0.254) (layer F.Cu) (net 9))
 (segment (start 69.088 49.784) (end 69.469 50.165) (width 0.254) (layer F.Cu) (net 9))
 (segment (start 69.088 40.64) (end 69.088 49.784) (width 0.254) (layer F.Cu) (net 9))
 (segment (start 69.342 40.386) (end 69.088 40.64) (width 0.254) (layer F.Cu) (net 9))
 (segment (start 78.359 42.926) (end 99.314 42.926) (width 0.254) (layer B.Cu) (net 4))
 (segment (start 101.6 53.34) (end 103.505 55.245) (width 0.254) (layer B.Cu) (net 4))
 (segment (start 101.6 45.212) (end 101.6 53.34) (width 0.254) (layer B.Cu) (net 4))
 (segment (start 99.314 42.926) (end 101.6 45.212) (width 0.254) (layer B.Cu) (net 4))
 (segment (start 103.505 55.245) (end 103.505 57.785) (width 0.254) (layer F.Cu) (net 4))
 (segment (start 103.505 62.865) (end 121.539 62.865) (width 0.254) (layer B.Cu) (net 21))
 (segment (start 121.539 62.865) (end 125.476 58.928) (width 0.254) (layer B.Cu) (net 21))
 (segment (start 75.819 42.926) (end 75.819 49.149) (width 0.254) (layer B.Cu) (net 6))
 (segment (start 75.819 49.149) (end 81.534 54.864) (width 0.254) (layer B.Cu) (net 6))
 (segment (start 81.534 54.864) (end 81.534 71.628) (width 0.254) (layer B.Cu) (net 6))
 (segment (start 81.534 71.628) (end 79.248 73.914) (width 0.254) (layer B.Cu) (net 6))
 (segment (start 81.534 54.864) (end 92.964 54.864) (width 0.254) (layer B.Cu) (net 6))
 (segment (start 92.964 54.864) (end 95.885 57.785) (width 0.254) (layer B.Cu) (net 6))
 (segment (start 77.089 40.386) (end 77.089 39.751) (width 0.254) (layer F.Cu) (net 5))
 (segment (start 98.044 58.166) (end 95.885 60.325) (width 0.254) (layer F.Cu) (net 5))
 (segment (start 98.044 41.148) (end 98.044 58.166) (width 0.254) (layer F.Cu) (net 5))
 (segment (start 96.012 39.116) (end 98.044 41.148) (width 0.254) (layer F.Cu) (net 5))
 (segment (start 77.724 39.116) (end 96.012 39.116) (width 0.254) (layer F.Cu) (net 5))
 (segment (start 77.089 39.751) (end 77.724 39.116) (width 0.254) (layer F.Cu) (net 5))
 (segment (start 125.476 37.592) (end 110.49 37.592) (width 2) (layer F.Cu) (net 18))
 (segment (start 110.49 37.592) (end 95.758 22.86) (width 2) (layer F.Cu) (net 18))
 (segment (start 125.476 37.592) (end 133.604 37.592) (width 2) (layer F.Cu) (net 18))
 (segment (start 133.604 37.592) (end 135.636 39.624) (width 2) (layer F.Cu) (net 18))
 (segment (start 135.636 39.624) (end 135.636 65.024) (width 2) (layer F.Cu) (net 18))
 (segment (start 135.636 65.024) (end 135.128 65.532) (width 2) (layer F.Cu) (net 18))
 (segment (start 135.128 65.532) (end 125.476 65.532) (width 2) (layer F.Cu) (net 18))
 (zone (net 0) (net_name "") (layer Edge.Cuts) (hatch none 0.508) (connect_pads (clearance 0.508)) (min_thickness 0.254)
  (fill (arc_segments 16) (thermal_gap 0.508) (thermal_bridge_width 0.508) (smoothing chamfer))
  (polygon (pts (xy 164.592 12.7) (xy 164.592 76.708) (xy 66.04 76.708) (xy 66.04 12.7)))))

